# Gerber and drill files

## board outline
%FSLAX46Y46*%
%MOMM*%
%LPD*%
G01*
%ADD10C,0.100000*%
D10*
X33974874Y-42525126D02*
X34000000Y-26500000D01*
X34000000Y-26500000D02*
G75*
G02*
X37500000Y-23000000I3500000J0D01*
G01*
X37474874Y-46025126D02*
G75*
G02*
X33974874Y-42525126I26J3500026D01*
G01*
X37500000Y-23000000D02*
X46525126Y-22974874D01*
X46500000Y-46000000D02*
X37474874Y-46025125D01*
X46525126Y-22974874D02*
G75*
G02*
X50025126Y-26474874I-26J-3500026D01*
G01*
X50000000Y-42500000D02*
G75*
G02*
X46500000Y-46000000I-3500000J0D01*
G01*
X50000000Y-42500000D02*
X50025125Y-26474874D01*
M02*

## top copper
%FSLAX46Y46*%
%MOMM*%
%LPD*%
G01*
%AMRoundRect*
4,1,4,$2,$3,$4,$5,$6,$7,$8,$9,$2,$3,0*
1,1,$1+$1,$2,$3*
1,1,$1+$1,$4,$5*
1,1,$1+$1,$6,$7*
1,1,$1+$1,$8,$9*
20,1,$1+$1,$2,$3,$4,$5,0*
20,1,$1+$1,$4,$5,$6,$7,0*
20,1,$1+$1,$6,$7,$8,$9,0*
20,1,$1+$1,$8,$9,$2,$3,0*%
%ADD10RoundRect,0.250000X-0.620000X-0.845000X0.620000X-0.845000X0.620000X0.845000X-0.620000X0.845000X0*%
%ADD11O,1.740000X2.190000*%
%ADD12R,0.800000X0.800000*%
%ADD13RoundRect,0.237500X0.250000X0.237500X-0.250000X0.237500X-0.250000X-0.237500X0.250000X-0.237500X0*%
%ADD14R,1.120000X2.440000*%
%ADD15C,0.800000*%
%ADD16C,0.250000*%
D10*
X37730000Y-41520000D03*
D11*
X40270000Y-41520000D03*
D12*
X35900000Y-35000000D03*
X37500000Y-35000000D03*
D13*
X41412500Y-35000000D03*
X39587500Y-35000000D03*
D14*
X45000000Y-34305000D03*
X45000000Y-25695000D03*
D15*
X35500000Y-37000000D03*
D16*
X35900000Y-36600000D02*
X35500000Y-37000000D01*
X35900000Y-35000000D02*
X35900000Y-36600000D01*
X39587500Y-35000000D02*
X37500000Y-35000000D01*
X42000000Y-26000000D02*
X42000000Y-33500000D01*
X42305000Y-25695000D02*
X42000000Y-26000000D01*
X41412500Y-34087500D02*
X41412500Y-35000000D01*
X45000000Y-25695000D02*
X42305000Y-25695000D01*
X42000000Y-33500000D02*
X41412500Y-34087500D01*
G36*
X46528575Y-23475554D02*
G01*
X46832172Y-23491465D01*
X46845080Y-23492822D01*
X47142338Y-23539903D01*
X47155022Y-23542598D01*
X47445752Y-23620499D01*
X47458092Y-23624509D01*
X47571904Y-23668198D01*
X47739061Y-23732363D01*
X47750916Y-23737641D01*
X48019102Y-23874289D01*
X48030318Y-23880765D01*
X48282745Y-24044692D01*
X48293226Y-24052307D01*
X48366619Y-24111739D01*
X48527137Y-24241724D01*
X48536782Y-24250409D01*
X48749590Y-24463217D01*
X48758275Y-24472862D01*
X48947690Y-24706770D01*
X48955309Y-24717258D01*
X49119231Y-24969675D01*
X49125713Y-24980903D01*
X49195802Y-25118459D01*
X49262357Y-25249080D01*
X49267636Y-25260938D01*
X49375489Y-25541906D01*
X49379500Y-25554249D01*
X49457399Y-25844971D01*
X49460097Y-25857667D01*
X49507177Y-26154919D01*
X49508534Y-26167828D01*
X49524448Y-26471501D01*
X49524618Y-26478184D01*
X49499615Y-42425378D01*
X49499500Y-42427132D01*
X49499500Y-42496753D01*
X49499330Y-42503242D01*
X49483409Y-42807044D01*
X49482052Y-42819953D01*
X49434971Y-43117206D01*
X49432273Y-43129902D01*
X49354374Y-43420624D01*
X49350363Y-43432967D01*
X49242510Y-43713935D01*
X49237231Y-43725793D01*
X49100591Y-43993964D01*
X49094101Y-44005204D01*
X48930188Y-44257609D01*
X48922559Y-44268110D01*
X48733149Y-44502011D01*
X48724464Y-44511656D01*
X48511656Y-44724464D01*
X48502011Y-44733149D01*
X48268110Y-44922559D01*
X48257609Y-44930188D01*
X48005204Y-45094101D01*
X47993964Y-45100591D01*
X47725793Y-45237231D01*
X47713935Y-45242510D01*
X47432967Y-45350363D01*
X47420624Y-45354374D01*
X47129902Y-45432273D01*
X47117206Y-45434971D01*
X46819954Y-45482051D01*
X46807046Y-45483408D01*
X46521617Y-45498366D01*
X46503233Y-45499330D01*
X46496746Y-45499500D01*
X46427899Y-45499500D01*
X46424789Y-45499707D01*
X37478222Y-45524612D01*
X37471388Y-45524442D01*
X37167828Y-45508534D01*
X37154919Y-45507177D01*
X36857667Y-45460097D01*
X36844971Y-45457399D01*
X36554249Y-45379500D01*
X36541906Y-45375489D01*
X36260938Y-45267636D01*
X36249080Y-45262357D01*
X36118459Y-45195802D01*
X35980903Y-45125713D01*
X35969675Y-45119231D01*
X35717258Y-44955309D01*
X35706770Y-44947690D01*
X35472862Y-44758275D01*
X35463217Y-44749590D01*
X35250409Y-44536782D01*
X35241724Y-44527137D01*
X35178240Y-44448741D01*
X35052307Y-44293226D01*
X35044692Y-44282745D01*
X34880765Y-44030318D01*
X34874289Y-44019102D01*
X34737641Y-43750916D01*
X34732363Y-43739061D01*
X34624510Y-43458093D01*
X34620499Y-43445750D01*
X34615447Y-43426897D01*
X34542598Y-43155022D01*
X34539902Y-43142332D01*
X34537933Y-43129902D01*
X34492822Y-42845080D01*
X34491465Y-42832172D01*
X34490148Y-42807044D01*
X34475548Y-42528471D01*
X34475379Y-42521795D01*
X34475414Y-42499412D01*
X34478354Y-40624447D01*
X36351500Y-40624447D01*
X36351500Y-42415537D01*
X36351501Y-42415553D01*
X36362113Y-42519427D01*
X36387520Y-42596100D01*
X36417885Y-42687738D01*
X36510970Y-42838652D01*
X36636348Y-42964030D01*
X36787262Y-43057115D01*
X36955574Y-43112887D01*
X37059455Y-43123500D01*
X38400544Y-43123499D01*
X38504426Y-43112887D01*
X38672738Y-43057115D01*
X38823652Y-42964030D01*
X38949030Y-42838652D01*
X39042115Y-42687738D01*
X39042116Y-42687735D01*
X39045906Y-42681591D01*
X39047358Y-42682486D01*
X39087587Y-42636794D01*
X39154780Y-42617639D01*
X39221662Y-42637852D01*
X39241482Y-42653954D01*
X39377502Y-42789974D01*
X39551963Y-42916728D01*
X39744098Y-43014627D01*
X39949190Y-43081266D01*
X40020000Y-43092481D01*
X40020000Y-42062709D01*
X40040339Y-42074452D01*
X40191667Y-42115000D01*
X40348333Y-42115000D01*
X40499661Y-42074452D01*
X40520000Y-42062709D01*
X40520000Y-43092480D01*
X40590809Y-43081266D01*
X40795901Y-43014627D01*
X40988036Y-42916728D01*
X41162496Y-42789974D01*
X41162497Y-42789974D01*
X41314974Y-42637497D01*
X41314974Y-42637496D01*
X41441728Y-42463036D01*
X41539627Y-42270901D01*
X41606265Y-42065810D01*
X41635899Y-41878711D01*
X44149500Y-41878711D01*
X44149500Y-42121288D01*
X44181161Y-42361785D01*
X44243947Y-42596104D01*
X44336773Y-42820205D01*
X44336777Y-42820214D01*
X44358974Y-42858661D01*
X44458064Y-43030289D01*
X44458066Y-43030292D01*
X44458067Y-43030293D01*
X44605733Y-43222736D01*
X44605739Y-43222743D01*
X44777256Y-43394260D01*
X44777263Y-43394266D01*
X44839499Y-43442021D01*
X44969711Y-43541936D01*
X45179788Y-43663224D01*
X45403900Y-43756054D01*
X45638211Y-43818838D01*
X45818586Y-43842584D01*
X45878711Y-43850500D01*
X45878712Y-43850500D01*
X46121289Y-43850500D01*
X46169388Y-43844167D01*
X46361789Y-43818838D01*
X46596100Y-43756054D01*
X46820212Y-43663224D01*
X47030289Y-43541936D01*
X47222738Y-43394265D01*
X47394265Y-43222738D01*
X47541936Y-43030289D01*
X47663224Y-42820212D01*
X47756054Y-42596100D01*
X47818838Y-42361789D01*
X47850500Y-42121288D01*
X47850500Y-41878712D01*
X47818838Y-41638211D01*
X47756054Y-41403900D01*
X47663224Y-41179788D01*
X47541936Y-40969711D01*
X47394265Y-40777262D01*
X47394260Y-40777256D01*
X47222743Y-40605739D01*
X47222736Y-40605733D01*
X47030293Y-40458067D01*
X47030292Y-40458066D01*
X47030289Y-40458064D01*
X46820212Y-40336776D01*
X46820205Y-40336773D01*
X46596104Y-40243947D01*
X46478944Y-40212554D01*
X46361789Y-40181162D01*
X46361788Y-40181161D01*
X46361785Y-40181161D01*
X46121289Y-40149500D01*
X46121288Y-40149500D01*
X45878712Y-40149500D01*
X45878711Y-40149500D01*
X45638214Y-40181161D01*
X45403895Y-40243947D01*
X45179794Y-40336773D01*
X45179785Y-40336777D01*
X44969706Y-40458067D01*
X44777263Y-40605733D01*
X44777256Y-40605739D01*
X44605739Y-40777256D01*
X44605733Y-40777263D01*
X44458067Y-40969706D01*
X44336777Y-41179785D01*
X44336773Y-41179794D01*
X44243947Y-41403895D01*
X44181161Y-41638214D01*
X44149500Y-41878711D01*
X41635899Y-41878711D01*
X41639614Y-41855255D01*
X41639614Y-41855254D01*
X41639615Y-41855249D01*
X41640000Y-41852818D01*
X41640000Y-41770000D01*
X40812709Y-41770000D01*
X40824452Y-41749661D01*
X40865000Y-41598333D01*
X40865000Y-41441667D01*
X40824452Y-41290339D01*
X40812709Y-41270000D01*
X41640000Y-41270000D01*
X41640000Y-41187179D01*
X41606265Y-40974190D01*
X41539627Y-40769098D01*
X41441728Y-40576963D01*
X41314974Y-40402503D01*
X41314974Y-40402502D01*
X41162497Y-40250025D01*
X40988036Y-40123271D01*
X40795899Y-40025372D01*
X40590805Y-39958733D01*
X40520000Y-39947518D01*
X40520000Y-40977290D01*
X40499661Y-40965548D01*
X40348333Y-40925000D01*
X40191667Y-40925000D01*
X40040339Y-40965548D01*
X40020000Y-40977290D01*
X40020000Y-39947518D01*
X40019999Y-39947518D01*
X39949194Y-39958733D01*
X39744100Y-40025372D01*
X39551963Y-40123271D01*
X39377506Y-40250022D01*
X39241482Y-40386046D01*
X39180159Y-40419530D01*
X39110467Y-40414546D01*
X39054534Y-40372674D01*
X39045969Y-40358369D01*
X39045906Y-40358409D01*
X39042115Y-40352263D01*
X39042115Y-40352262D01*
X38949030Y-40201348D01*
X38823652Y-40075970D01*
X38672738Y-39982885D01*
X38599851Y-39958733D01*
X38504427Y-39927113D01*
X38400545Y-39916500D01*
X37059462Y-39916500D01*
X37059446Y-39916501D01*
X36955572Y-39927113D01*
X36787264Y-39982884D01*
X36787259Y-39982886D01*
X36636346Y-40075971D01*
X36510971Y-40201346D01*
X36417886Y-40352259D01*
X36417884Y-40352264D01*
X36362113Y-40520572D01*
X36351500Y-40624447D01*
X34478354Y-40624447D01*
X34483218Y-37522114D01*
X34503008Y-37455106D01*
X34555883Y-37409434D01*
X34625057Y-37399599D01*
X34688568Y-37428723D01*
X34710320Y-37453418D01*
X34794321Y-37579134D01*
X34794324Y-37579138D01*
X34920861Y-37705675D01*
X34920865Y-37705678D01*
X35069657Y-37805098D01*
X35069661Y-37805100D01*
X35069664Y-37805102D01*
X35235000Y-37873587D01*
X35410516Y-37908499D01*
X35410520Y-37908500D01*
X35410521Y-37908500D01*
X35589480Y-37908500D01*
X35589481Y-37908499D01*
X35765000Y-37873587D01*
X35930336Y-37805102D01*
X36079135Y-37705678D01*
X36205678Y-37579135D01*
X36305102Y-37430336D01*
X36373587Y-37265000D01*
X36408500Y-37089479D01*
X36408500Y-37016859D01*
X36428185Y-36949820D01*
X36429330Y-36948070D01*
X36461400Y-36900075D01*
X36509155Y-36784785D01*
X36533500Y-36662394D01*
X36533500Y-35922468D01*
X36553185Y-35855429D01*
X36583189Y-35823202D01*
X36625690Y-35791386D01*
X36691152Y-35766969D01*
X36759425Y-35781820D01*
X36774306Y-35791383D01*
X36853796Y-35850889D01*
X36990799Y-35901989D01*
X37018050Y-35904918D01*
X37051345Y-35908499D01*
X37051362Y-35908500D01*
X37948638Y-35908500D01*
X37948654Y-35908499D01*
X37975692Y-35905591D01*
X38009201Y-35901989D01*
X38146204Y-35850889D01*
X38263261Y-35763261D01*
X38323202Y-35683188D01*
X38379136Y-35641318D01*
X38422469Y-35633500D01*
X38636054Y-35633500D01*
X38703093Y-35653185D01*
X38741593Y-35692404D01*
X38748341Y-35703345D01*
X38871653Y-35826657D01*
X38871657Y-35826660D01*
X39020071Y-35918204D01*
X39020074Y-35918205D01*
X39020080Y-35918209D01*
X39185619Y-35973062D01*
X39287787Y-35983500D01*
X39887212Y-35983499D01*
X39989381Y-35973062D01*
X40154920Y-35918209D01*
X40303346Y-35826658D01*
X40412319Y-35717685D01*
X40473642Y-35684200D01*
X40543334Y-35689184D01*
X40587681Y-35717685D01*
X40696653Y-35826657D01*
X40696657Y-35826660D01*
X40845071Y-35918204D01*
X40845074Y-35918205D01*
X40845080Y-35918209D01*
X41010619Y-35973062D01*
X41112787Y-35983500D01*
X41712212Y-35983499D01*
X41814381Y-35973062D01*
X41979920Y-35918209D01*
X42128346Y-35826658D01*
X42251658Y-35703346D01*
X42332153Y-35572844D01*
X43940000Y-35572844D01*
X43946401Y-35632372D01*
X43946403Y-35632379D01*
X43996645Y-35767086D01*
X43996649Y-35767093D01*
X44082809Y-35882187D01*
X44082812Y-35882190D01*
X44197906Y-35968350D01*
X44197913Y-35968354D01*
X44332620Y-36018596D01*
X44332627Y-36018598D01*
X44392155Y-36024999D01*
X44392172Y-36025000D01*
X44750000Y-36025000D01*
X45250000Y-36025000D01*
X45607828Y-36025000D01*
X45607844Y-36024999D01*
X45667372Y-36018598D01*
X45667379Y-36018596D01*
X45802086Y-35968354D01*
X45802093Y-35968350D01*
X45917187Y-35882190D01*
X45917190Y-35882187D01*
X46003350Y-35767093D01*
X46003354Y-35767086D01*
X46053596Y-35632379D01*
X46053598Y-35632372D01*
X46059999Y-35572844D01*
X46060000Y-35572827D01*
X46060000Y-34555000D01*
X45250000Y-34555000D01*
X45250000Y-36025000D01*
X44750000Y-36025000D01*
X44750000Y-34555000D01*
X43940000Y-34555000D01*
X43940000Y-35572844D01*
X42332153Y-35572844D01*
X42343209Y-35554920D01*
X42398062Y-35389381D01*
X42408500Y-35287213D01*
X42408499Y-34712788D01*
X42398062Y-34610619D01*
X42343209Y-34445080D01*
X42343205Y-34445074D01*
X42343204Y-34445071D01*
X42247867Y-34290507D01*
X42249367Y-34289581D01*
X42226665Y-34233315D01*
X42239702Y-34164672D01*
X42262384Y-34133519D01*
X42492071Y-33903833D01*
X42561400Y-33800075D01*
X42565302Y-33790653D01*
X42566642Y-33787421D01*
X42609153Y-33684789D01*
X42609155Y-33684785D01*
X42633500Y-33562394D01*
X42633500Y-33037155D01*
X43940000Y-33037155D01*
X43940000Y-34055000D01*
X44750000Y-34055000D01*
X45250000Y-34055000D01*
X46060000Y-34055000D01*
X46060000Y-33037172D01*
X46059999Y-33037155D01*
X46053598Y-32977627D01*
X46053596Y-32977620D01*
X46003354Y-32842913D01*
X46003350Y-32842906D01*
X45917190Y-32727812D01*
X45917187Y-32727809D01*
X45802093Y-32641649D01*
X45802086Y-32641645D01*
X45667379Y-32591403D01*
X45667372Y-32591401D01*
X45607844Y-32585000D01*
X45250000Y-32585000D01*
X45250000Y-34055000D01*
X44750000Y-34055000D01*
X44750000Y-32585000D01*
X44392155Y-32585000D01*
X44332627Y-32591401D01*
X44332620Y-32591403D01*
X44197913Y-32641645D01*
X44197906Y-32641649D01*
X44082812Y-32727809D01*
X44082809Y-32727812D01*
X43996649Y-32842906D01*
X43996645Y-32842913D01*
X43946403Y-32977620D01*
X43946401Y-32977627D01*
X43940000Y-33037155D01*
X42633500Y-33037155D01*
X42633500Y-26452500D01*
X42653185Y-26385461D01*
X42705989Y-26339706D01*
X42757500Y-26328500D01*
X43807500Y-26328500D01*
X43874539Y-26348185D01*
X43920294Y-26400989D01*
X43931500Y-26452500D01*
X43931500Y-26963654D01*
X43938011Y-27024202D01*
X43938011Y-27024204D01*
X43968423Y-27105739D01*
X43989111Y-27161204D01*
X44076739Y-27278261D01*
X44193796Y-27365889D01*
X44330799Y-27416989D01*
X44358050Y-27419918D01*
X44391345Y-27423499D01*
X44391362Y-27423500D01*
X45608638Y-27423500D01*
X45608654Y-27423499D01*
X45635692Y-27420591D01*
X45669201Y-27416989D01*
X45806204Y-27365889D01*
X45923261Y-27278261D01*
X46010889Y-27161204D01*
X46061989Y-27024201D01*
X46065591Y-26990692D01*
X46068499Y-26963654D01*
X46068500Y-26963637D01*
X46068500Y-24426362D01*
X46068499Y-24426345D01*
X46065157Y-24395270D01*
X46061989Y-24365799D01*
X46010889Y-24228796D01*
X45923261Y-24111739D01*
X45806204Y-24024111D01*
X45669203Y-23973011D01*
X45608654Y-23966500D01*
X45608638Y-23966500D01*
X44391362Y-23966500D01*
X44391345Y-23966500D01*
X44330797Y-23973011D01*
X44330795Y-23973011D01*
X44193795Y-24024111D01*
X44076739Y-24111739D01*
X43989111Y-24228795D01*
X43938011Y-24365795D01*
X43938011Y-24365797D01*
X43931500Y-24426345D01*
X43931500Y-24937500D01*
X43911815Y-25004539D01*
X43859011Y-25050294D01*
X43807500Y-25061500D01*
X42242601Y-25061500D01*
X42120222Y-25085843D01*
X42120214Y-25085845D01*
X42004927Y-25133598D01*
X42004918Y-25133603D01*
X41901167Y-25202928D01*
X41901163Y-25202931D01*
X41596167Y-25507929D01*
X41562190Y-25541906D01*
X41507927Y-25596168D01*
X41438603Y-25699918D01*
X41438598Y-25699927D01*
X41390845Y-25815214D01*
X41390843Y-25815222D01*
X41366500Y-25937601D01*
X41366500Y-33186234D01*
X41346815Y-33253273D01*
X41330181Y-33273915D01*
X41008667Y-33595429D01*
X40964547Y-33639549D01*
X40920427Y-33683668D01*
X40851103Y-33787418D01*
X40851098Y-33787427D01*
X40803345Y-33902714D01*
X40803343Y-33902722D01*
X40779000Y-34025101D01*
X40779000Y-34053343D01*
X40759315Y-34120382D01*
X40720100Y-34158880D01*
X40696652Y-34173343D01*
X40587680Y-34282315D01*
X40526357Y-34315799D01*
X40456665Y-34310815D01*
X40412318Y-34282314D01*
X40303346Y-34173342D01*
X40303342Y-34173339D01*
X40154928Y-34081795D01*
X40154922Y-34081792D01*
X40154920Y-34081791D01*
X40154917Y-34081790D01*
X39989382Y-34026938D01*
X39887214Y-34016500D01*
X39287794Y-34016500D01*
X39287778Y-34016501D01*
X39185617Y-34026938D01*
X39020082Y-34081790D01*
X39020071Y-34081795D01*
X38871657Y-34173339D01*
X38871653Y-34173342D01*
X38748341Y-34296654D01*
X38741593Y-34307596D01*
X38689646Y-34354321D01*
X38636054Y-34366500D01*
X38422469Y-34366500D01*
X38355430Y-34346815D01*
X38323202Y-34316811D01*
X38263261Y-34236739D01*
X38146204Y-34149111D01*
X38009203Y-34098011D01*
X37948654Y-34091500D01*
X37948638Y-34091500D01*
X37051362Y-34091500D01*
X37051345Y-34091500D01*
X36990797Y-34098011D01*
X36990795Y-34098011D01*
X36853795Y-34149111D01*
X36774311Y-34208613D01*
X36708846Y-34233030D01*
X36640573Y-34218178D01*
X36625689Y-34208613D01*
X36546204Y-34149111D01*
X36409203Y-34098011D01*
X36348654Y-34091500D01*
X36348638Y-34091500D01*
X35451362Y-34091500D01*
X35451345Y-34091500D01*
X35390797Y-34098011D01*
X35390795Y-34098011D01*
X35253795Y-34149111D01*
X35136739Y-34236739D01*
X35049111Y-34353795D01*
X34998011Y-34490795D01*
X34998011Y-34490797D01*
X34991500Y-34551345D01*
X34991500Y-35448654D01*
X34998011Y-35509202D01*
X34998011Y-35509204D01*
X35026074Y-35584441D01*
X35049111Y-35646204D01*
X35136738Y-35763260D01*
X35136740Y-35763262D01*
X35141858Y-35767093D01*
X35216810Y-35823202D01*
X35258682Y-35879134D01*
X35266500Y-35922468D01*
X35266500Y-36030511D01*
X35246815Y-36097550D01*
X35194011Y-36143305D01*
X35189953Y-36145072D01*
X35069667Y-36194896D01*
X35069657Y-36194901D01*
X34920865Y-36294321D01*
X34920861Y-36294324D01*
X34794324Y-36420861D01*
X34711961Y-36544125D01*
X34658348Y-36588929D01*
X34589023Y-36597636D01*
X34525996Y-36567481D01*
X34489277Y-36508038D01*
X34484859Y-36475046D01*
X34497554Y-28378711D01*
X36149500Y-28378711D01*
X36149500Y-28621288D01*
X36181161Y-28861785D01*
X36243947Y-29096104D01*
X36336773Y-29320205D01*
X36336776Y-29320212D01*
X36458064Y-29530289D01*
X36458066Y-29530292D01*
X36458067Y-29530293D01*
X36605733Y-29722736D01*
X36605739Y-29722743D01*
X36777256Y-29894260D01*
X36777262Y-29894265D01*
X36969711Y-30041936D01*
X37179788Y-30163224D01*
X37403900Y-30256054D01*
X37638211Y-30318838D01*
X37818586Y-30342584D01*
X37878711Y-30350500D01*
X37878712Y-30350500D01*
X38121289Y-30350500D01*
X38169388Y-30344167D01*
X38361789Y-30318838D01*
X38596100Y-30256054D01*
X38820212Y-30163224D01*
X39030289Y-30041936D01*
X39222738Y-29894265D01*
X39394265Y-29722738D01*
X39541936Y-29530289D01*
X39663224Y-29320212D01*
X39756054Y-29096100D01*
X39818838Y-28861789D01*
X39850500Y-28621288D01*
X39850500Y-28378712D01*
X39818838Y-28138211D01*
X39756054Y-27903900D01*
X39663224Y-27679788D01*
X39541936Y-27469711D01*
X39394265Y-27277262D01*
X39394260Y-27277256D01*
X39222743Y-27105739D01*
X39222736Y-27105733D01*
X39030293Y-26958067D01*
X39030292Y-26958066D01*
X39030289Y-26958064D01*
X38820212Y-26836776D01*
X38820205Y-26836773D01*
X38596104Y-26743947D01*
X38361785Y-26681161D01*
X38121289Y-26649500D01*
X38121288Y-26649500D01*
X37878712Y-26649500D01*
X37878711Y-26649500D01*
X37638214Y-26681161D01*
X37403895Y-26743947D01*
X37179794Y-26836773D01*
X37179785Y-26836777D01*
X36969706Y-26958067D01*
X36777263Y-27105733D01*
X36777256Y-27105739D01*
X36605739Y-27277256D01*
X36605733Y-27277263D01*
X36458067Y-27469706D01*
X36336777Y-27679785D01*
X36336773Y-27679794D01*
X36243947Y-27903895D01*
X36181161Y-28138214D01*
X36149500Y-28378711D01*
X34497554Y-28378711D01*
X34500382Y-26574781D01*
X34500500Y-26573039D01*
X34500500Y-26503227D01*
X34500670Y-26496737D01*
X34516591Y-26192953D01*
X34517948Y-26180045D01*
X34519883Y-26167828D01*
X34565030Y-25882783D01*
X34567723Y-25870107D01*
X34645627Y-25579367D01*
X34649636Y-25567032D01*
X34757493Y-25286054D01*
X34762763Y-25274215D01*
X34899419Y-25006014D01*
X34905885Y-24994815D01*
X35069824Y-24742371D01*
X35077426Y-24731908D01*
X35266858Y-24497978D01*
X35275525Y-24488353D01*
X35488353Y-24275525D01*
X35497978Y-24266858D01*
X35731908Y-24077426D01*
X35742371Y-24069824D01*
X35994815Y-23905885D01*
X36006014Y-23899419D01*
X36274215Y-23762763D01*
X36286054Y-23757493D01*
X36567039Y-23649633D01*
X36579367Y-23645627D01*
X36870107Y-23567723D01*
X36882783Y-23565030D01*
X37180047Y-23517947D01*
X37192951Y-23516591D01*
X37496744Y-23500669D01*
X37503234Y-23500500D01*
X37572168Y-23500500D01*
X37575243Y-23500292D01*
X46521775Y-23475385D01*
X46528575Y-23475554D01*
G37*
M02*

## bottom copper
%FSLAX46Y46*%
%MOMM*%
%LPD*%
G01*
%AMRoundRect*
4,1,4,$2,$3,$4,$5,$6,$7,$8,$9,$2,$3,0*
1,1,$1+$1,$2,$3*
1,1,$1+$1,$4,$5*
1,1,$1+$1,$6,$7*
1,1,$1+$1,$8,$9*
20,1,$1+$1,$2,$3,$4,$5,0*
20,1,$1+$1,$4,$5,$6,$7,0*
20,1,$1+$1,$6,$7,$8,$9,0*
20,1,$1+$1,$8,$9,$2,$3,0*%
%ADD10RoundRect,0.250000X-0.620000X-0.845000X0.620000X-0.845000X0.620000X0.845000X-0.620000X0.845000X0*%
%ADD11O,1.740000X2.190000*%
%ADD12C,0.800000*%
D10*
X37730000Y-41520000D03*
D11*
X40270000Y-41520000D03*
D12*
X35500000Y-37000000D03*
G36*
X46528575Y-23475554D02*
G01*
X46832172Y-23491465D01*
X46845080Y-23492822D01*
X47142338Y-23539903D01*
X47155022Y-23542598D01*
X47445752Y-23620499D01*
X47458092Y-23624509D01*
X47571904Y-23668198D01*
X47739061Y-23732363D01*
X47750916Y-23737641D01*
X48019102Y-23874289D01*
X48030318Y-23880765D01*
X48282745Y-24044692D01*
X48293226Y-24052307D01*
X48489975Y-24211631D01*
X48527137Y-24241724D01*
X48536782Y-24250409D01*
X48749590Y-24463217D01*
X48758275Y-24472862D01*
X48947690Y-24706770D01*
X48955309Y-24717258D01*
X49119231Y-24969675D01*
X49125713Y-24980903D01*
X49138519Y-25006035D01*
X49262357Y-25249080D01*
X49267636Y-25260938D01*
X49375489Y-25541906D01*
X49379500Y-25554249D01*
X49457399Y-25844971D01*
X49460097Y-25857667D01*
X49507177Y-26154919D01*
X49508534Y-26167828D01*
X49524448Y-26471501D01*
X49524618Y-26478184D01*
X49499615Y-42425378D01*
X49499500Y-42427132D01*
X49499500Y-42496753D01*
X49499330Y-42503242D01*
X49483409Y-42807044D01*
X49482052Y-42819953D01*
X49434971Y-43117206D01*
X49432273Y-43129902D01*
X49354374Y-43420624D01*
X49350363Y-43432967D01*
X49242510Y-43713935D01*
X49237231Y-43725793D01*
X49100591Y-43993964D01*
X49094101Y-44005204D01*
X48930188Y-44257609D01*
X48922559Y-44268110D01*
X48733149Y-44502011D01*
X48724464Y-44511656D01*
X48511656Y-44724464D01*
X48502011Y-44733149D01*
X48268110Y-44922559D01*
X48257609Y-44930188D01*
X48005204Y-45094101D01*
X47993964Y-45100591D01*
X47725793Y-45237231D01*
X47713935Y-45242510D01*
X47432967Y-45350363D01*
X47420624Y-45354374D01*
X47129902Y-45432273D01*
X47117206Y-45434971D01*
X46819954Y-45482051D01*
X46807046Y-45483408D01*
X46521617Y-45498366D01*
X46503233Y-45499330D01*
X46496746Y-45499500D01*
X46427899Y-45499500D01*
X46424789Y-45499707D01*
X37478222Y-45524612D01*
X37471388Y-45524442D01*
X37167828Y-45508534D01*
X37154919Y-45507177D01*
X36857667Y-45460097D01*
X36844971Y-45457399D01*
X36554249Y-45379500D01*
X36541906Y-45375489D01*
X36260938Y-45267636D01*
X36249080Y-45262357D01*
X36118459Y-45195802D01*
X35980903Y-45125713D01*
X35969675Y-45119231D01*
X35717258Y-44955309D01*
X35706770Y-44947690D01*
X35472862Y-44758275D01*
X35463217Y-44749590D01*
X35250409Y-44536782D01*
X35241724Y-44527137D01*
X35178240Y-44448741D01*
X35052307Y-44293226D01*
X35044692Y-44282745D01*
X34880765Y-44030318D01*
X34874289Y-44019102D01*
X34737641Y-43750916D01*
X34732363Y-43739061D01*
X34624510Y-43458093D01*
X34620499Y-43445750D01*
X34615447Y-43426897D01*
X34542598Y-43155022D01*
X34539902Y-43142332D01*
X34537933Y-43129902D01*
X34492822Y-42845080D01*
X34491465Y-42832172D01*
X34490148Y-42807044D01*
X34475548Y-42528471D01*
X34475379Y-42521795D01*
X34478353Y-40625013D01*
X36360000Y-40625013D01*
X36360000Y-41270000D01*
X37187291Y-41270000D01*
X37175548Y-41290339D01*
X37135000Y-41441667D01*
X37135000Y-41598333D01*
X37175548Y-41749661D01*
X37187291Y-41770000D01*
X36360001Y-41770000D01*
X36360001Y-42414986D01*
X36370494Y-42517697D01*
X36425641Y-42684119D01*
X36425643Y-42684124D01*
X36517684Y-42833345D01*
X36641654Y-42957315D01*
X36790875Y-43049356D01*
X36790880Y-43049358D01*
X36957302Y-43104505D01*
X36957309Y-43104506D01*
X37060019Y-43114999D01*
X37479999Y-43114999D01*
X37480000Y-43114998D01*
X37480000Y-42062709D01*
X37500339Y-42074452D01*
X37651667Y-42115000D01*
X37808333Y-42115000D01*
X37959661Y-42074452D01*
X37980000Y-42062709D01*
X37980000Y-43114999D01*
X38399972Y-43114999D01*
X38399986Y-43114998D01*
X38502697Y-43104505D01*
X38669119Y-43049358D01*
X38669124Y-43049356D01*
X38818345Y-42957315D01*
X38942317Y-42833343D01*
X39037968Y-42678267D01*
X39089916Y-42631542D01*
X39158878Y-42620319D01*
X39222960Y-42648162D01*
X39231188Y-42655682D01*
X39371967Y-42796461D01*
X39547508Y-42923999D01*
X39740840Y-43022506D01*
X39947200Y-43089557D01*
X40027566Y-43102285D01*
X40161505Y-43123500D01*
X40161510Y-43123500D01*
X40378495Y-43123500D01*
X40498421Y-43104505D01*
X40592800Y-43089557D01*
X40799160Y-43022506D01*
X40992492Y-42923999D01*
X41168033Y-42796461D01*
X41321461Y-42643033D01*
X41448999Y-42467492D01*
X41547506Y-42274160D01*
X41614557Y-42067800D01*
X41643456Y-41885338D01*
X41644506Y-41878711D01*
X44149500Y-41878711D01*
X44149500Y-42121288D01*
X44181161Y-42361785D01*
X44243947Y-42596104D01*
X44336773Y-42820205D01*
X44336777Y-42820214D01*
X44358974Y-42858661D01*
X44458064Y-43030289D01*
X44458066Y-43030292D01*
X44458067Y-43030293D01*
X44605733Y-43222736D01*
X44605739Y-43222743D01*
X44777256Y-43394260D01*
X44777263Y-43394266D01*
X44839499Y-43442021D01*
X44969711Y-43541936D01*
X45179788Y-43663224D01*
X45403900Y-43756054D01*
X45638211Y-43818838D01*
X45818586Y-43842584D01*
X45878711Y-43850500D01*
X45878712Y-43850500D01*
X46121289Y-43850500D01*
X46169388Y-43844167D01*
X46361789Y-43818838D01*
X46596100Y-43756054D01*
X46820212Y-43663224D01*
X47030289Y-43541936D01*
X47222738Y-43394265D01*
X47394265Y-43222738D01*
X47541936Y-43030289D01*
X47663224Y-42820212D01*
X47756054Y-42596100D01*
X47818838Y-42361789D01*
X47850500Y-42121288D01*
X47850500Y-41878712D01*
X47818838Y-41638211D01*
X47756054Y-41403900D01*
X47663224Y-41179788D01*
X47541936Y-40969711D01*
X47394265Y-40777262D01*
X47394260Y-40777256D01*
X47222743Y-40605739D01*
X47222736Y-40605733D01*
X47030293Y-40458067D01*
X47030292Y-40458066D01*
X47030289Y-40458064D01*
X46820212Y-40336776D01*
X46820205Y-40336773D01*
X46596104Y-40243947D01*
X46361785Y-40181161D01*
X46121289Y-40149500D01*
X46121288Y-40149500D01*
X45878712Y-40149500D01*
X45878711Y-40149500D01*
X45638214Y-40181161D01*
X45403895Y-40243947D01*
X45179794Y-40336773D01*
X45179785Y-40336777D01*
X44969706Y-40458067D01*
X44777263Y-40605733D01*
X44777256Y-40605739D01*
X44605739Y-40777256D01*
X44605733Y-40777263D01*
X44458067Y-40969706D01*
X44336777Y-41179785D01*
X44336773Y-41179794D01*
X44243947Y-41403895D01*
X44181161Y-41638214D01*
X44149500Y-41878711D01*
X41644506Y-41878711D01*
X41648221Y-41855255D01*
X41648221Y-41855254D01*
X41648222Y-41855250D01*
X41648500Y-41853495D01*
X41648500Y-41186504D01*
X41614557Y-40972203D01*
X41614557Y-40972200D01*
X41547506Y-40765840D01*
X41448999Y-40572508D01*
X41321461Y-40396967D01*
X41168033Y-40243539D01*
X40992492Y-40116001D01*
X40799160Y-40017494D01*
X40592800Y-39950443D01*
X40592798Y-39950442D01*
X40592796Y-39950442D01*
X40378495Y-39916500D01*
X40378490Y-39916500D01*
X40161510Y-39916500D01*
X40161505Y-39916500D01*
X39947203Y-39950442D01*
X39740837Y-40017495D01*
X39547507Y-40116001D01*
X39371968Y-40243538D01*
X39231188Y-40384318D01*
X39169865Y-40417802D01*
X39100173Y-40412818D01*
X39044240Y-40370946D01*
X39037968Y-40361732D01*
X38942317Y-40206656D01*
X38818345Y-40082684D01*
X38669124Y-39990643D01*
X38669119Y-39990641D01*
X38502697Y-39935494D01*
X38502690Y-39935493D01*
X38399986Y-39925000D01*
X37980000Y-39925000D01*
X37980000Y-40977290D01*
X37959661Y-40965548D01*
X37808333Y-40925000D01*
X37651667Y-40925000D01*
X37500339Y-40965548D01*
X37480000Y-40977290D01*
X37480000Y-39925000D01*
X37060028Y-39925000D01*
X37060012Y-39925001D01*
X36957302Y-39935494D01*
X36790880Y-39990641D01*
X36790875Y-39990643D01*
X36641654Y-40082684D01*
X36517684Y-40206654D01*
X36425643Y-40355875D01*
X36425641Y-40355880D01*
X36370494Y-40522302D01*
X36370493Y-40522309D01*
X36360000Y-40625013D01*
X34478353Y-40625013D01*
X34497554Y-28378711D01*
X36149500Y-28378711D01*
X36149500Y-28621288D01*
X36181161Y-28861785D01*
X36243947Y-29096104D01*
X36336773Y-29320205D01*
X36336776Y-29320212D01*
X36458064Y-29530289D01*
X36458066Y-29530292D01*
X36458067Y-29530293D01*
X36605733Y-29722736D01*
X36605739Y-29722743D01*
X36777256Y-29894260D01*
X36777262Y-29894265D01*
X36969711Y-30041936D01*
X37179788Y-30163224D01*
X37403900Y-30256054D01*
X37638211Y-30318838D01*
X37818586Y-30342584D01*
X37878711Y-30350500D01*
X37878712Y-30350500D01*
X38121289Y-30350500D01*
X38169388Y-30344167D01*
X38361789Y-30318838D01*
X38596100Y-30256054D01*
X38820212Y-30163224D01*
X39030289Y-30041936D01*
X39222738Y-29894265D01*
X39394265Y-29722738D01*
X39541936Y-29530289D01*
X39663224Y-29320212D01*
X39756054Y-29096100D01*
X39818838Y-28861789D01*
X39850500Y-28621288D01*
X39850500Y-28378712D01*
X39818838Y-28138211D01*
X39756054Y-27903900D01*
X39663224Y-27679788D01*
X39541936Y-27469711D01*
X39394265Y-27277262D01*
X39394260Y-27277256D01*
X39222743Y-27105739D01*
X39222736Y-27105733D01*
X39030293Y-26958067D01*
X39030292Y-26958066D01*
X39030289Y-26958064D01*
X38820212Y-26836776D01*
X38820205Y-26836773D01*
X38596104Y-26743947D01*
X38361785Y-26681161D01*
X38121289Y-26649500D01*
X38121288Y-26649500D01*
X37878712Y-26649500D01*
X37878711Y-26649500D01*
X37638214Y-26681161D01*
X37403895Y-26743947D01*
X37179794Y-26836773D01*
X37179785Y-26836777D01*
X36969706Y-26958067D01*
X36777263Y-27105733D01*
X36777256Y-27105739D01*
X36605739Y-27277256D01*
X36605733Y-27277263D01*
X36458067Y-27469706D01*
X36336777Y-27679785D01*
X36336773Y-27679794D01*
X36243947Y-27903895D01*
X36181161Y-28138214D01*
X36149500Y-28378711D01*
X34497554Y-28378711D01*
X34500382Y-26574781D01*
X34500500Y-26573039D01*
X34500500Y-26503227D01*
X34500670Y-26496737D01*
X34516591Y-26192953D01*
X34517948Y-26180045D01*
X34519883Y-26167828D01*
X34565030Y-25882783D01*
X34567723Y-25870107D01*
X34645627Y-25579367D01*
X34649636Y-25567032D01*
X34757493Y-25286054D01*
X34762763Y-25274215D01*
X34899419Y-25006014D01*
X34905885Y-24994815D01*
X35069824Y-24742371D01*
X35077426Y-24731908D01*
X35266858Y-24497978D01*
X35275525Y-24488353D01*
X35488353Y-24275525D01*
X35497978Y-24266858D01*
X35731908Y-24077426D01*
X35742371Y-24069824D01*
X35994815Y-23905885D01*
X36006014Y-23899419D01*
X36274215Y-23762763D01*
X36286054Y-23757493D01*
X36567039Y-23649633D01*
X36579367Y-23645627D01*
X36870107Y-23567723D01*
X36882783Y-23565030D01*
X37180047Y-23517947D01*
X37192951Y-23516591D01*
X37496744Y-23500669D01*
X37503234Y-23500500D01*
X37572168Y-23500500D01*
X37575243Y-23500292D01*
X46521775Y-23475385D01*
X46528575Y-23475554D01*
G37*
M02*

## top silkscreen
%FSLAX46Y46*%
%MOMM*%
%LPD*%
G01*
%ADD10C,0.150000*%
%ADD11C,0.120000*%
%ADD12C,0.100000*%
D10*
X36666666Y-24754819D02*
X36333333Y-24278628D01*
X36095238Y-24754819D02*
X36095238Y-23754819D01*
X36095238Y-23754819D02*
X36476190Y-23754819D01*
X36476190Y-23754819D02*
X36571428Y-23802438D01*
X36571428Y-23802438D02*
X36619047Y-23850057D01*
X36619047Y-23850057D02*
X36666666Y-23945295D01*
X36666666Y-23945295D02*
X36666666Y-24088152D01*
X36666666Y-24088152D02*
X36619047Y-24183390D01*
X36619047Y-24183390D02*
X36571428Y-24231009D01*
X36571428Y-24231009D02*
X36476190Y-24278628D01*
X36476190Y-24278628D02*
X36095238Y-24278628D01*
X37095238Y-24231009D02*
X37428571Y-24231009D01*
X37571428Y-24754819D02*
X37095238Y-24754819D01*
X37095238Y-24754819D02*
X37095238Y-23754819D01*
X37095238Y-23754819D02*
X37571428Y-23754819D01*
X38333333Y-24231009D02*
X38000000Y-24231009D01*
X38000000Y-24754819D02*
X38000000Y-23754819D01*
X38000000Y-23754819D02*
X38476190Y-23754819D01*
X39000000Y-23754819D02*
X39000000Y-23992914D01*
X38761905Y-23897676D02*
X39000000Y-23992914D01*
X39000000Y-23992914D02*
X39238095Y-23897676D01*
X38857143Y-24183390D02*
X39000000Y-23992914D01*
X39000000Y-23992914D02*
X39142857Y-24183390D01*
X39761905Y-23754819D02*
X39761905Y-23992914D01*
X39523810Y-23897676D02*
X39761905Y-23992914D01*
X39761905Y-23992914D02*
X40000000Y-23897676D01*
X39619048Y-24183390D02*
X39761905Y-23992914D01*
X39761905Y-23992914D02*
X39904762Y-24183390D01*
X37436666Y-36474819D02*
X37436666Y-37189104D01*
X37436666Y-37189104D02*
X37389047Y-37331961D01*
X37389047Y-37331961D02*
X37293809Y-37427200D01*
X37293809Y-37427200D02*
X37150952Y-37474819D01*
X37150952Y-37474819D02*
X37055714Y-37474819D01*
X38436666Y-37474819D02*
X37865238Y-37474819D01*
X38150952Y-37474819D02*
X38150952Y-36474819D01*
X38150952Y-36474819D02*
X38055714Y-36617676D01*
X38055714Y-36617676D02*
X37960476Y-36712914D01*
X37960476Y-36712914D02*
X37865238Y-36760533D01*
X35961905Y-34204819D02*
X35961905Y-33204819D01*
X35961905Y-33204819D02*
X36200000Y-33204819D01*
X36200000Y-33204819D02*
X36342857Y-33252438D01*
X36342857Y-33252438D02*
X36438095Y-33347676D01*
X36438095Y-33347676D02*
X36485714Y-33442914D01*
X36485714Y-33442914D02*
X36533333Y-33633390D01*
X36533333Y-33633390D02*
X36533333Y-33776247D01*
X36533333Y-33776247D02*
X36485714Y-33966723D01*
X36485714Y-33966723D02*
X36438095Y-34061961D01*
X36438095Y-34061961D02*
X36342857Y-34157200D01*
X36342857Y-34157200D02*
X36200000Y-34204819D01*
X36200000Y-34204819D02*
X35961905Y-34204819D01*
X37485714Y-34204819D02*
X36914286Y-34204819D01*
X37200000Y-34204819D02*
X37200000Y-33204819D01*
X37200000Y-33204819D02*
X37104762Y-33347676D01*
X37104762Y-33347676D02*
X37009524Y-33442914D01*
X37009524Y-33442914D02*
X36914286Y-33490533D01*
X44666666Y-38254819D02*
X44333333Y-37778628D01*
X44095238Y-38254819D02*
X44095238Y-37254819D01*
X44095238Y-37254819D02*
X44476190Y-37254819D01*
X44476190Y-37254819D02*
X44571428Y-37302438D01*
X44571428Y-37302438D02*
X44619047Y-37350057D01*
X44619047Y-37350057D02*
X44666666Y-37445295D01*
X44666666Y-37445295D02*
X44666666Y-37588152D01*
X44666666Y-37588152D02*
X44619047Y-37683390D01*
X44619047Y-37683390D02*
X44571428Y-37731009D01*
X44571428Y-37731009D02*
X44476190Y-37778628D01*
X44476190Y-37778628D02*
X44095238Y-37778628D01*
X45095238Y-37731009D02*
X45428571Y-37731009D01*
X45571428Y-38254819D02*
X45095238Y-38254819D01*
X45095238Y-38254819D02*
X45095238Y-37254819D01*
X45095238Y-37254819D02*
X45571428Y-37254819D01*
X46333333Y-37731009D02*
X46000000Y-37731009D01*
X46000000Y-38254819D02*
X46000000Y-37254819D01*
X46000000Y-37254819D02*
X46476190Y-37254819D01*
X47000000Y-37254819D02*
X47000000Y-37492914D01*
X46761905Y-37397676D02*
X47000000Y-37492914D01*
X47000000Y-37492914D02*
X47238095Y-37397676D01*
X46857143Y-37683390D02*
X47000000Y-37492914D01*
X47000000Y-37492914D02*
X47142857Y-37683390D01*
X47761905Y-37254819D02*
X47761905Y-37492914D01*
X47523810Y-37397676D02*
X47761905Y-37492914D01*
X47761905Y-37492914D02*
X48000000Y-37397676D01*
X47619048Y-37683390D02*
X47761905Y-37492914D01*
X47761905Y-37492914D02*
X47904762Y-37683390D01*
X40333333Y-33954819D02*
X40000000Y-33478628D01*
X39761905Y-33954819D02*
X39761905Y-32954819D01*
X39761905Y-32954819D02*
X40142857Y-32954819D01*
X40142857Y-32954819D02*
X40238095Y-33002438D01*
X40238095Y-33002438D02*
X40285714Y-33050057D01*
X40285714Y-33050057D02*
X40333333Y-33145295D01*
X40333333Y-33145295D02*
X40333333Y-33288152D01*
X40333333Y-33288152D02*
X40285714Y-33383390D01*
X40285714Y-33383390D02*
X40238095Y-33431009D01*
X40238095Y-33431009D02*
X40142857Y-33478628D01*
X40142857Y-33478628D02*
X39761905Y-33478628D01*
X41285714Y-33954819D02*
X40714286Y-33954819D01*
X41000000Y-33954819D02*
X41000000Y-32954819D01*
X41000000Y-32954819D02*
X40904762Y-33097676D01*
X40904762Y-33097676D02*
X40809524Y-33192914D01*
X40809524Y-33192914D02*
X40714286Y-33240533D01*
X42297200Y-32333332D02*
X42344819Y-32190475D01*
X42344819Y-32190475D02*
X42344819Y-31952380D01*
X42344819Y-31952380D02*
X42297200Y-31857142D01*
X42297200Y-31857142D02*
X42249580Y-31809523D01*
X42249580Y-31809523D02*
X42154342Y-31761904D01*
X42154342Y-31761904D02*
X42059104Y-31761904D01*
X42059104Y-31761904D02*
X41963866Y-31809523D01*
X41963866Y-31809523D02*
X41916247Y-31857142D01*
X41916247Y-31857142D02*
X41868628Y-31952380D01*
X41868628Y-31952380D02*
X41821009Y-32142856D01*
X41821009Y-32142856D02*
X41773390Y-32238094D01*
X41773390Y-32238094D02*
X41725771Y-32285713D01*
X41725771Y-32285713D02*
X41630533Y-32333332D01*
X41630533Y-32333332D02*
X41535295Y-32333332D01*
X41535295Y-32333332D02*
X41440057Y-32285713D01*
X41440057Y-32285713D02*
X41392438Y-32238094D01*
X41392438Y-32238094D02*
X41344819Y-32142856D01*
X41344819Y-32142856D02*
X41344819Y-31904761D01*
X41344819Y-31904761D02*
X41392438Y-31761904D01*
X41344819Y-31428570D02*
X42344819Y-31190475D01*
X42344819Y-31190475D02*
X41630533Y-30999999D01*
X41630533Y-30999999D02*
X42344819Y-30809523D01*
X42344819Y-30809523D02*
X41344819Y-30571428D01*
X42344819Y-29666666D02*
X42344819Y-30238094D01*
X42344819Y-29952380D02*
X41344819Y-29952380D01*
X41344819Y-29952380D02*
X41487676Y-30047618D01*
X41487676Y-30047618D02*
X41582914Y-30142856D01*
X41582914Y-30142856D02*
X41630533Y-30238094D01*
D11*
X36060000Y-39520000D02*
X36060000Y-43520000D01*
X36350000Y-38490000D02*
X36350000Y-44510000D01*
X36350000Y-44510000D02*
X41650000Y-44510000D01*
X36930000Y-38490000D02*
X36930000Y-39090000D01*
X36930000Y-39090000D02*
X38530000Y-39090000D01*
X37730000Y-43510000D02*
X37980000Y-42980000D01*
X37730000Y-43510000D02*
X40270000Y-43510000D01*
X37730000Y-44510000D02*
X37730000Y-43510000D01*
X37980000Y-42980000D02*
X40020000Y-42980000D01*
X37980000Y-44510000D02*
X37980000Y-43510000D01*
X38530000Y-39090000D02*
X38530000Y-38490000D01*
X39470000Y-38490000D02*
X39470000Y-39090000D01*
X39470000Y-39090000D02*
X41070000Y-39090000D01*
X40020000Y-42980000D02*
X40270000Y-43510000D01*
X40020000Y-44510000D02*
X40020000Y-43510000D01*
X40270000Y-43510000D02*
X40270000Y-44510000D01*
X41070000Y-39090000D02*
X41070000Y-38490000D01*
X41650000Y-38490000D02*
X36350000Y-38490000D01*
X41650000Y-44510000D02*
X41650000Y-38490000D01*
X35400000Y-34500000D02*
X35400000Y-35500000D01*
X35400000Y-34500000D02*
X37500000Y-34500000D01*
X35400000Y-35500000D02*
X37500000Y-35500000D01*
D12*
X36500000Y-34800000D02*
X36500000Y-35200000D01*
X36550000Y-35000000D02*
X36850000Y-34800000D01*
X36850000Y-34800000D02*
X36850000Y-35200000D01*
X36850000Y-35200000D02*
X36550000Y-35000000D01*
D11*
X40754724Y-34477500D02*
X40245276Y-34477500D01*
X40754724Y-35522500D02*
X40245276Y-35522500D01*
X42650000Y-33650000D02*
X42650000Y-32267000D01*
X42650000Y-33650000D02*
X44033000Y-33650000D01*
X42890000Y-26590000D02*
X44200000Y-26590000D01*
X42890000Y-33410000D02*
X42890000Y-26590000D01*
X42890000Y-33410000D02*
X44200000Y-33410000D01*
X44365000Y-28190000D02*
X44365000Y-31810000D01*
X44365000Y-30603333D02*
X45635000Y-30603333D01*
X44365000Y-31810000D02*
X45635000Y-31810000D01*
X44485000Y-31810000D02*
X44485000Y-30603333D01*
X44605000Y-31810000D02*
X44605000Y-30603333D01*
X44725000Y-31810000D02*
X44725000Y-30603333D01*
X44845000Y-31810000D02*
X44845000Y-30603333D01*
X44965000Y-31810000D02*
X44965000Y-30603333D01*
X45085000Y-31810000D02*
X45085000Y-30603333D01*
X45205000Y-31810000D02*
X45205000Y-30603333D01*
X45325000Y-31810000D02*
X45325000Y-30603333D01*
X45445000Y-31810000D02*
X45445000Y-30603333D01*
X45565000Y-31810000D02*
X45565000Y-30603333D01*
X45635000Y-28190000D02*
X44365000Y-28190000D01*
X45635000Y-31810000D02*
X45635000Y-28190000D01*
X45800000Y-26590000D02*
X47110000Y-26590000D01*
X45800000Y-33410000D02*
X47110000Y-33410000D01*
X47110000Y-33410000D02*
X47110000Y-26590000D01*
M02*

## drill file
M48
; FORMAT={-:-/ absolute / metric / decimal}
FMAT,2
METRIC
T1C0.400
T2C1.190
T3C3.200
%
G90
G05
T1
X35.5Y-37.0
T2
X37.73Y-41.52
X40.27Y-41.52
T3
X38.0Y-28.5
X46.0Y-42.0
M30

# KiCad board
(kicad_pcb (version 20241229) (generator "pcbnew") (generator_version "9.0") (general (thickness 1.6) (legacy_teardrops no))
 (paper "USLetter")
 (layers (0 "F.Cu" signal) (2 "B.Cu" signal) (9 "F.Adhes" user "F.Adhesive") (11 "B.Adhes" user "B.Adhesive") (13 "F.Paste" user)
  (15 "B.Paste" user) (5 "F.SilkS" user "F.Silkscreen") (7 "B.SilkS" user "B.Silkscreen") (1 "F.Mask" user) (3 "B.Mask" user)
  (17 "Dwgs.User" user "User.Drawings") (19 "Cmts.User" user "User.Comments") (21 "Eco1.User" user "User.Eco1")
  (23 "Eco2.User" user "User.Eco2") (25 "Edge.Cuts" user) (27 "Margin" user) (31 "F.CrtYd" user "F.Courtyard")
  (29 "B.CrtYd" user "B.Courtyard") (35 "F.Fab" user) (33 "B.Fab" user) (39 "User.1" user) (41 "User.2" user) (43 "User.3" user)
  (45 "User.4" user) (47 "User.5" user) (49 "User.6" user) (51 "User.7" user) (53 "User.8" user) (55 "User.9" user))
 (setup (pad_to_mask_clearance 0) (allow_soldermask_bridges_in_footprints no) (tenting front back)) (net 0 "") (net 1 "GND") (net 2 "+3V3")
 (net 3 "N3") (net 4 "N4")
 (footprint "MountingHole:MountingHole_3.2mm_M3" (layer "F.Cu") (at 38 28.5)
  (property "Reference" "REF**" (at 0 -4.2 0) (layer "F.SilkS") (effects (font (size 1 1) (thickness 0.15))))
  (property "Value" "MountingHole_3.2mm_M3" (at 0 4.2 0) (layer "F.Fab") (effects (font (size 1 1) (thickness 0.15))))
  (pad "" np_thru_hole circle (at 0 0) (size 3.2 3.2) (drill 3.2) (layers "*.Cu" "*.Mask")))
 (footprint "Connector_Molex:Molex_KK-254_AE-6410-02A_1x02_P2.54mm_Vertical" (layer "F.Cu") (at 37.73 41.52)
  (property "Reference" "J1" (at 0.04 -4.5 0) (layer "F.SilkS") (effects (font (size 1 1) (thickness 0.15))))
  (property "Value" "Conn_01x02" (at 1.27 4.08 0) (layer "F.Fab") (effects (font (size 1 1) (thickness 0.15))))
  (fp_line (start -1.67 -2) (end -1.67 2) (stroke (width 0.12) (type solid)) (layer "F.SilkS"))
  (fp_line (start -1.38 -3.03) (end -1.38 2.99) (stroke (width 0.12) (type solid)) (layer "F.SilkS"))
  (fp_line (start -1.38 2.99) (end 3.92 2.99) (stroke (width 0.12) (type solid)) (layer "F.SilkS"))
  (fp_line (start -0.8 -3.03) (end -0.8 -2.43) (stroke (width 0.12) (type solid)) (layer "F.SilkS"))
  (fp_line (start -0.8 -2.43) (end 0.8 -2.43) (stroke (width 0.12) (type solid)) (layer "F.SilkS"))
  (fp_line (start 0 1.99) (end 0.25 1.46) (stroke (width 0.12) (type solid)) (layer "F.SilkS"))
  (fp_line (start 0 1.99) (end 2.54 1.99) (stroke (width 0.12) (type solid)) (layer "F.SilkS"))
  (fp_line (start 0 2.99) (end 0 1.99) (stroke (width 0.12) (type solid)) (layer "F.SilkS"))
  (fp_line (start 0.25 1.46) (end 2.29 1.46) (stroke (width 0.12) (type solid)) (layer "F.SilkS"))
  (fp_line (start 0.25 2.99) (end 0.25 1.99) (stroke (width 0.12) (type solid)) (layer "F.SilkS"))
  (fp_line (start 0.8 -2.43) (end 0.8 -3.03) (stroke (width 0.12) (type solid)) (layer "F.SilkS"))
  (fp_line (start 1.74 -3.03) (end 1.74 -2.43) (stroke (width 0.12) (type solid)) (layer "F.SilkS"))
  (fp_line (start 1.74 -2.43) (end 3.34 -2.43) (stroke (width 0.12) (type solid)) (layer "F.SilkS"))
  (fp_line (start 2.29 1.46) (end 2.54 1.99) (stroke (width 0.12) (type solid)) (layer "F.SilkS"))
  (fp_line (start 2.29 2.99) (end 2.29 1.99) (stroke (width 0.12) (type solid)) (layer "F.SilkS"))
  (fp_line (start 2.54 1.99) (end 2.54 2.99) (stroke (width 0.12) (type solid)) (layer "F.SilkS"))
  (fp_line (start 3.34 -2.43) (end 3.34 -3.03) (stroke (width 0.12) (type solid)) (layer "F.SilkS"))
  (fp_line (start 3.92 -3.03) (end -1.38 -3.03) (stroke (width 0.12) (type solid)) (layer "F.SilkS"))
  (fp_line (start 3.92 2.99) (end 3.92 -3.03) (stroke (width 0.12) (type solid)) (layer "F.SilkS"))
  (pad "1" thru_hole roundrect (at 0 0) (size 1.74 2.19) (drill 1.19) (layers "*.Cu" "*.Mask") (remove_unused_layers no)
   (roundrect_rratio 0.143678) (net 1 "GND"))
  (pad "2" thru_hole oval (at 2.54 0) (size 1.74 2.19) (drill 1.19) (layers "*.Cu" "*.Mask") (remove_unused_layers no) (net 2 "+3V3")))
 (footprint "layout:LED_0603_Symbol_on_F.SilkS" (layer "F.Cu") (at 36.7 35)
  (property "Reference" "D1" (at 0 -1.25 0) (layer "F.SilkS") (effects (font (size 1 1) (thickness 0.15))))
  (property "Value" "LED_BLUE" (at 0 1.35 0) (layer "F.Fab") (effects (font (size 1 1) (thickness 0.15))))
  (fp_line (start -1.3 -0.5) (end -1.3 0.5) (stroke (width 0.12) (type solid)) (layer "F.SilkS"))
  (fp_line (start -1.3 -0.5) (end 0.8 -0.5) (stroke (width 0.12) (type solid)) (layer "F.SilkS"))
  (fp_line (start -1.3 0.5) (end 0.8 0.5) (stroke (width 0.12) (type solid)) (layer "F.SilkS"))
  (fp_line (start -0.2 -0.2) (end -0.2 0.2) (stroke (width 0.1) (type solid)) (layer "F.SilkS"))
  (fp_line (start -0.15 0) (end 0.15 -0.2) (stroke (width 0.1) (type solid)) (layer "F.SilkS"))
  (fp_line (start 0.15 -0.2) (end 0.15 0.2) (stroke (width 0.1) (type solid)) (layer "F.SilkS"))
  (fp_line (start 0.15 0.2) (end -0.15 0) (stroke (width 0.1) (type solid)) (layer "F.SilkS"))
  (pad "1" smd rect (at -0.8 0 180) (size 0.8 0.8) (layers "F.Cu" "F.Mask" "F.Paste") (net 1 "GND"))
  (pad "2" smd rect (at 0.8 0 180) (size 0.8 0.8) (layers "F.Cu" "F.Mask" "F.Paste") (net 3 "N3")))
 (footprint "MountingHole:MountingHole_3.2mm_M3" (layer "F.Cu") (at 46 42)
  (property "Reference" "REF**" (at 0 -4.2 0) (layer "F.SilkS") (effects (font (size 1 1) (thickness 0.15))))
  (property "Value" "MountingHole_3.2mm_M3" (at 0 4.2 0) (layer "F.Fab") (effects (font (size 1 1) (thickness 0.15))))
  (pad "" np_thru_hole circle (at 0 0) (size 3.2 3.2) (drill 3.2) (layers "*.Cu" "*.Mask")))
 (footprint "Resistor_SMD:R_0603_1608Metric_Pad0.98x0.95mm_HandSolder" (layer "F.Cu") (at 40.5 35 180)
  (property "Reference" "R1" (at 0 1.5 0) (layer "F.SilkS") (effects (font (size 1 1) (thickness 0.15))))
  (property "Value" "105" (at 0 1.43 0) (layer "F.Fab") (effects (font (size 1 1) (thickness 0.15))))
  (fp_line (start -0.254724 0.5225) (end 0.254724 0.5225) (stroke (width 0.12) (type solid)) (layer "F.SilkS"))
  (fp_line (start -0.254724 -0.5225) (end 0.254724 -0.5225) (stroke (width 0.12) (type solid)) (layer "F.SilkS"))
  (pad "1" smd roundrect (at -0.9125 0 180) (size 0.975 0.95) (layers "F.Cu" "F.Mask" "F.Paste") (roundrect_rratio 0.25) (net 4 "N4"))
  (pad "2" smd roundrect (at 0.9125 0 180) (size 0.975 0.95) (layers "F.Cu" "F.Mask" "F.Paste") (roundrect_rratio 0.25) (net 3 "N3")))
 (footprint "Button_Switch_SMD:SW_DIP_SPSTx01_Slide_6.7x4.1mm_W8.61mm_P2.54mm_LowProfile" (layer "F.Cu") (at 45 30 90)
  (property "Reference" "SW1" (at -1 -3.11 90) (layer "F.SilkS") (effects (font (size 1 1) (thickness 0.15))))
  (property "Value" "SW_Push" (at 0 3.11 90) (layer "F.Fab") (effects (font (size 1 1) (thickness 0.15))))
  (fp_line (start -3.65 -2.35) (end -2.267 -2.35) (stroke (width 0.12) (type solid)) (layer "F.SilkS"))
  (fp_line (start -3.65 -2.35) (end -3.65 -0.967) (stroke (width 0.12) (type solid)) (layer "F.SilkS"))
  (fp_line (start 3.41 -2.11) (end 3.41 -0.8) (stroke (width 0.12) (type solid)) (layer "F.SilkS"))
  (fp_line (start -3.41 -2.11) (end 3.41 -2.11) (stroke (width 0.12) (type solid)) (layer "F.SilkS"))
  (fp_line (start -3.41 -2.11) (end -3.41 -0.8) (stroke (width 0.12) (type solid)) (layer "F.SilkS"))
  (fp_line (start 1.81 -0.635) (end -1.81 -0.635) (stroke (width 0.12) (type solid)) (layer "F.SilkS"))
  (fp_line (start -0.603333 -0.635) (end -0.603333 0.635) (stroke (width 0.12) (type solid)) (layer "F.SilkS"))
  (fp_line (start -1.81 -0.635) (end -1.81 0.635) (stroke (width 0.12) (type solid)) (layer "F.SilkS"))
  (fp_line (start -1.81 -0.515) (end -0.603333 -0.515) (stroke (width 0.12) (type solid)) (layer "F.SilkS"))
  (fp_line (start -1.81 -0.395) (end -0.603333 -0.395) (stroke (width 0.12) (type solid)) (layer "F.SilkS"))
  (fp_line (start -1.81 -0.275) (end -0.603333 -0.275) (stroke (width 0.12) (type solid)) (layer "F.SilkS"))
  (fp_line (start -1.81 -0.155) (end -0.603333 -0.155) (stroke (width 0.12) (type solid)) (layer "F.SilkS"))
  (fp_line (start -1.81 -0.035) (end -0.603333 -0.035) (stroke (width 0.12) (type solid)) (layer "F.SilkS"))
  (fp_line (start -1.81 0.085) (end -0.603333 0.085) (stroke (width 0.12) (type solid)) (layer "F.SilkS"))
  (fp_line (start -1.81 0.205) (end -0.603333 0.205) (stroke (width 0.12) (type solid)) (layer "F.SilkS"))
  (fp_line (start -1.81 0.325) (end -0.603333 0.325) (stroke (width 0.12) (type solid)) (layer "F.SilkS"))
  (fp_line (start -1.81 0.445) (end -0.603333 0.445) (stroke (width 0.12) (type solid)) (layer "F.SilkS"))
  (fp_line (start -1.81 0.565) (end -0.603333 0.565) (stroke (width 0.12) (type solid)) (layer "F.SilkS"))
  (fp_line (start 1.81 0.635) (end 1.81 -0.635) (stroke (width 0.12) (type solid)) (layer "F.SilkS"))
  (fp_line (start -1.81 0.635) (end 1.81 0.635) (stroke (width 0.12) (type solid)) (layer "F.SilkS"))
  (fp_line (start 3.41 0.8) (end 3.41 2.11) (stroke (width 0.12) (type solid)) (layer "F.SilkS"))
  (fp_line (start -3.41 0.8) (end -3.41 2.11) (stroke (width 0.12) (type solid)) (layer "F.SilkS"))
  (fp_line (start -3.41 2.11) (end 3.41 2.11) (stroke (width 0.12) (type solid)) (layer "F.SilkS"))
  (pad "1" smd rect (at -4.305 0 90) (size 2.44 1.12) (layers "F.Cu" "F.Mask" "F.Paste") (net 2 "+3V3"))
  (pad "2" smd rect (at 4.305 0 90) (size 2.44 1.12) (layers "F.Cu" "F.Mask" "F.Paste") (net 4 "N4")))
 (gr_line (start 33.974874 42.525126) (end 34 26.5) (stroke (width 0.1) (type default)) (layer "Edge.Cuts"))
 (gr_arc (start 34 26.5) (mid 35.025126 24.025126) (end 37.5 23) (stroke (width 0.1) (type default)) (layer "Edge.Cuts"))
 (gr_arc (start 37.474874 46.025126) (mid 35 45) (end 33.974874 42.525126) (stroke (width 0.1) (type default)) (layer "Edge.Cuts"))
 (gr_line (start 37.5 23) (end 46.525126 22.974874) (stroke (width 0.1) (type default)) (layer "Edge.Cuts"))
 (gr_line (start 46.5 46) (end 37.474874 46.025125) (stroke (width 0.1) (type default)) (layer "Edge.Cuts"))
 (gr_arc (start 46.525126 22.974874) (mid 49 24) (end 50.025126 26.474874) (stroke (width 0.1) (type default)) (layer "Edge.Cuts"))
 (gr_arc (start 50 42.5) (mid 48.974874 44.974874) (end 46.5 46) (stroke (width 0.1) (type default)) (layer "Edge.Cuts"))
 (gr_line (start 50 42.5) (end 50.025125 26.474874) (stroke (width 0.1) (type default)) (layer "Edge.Cuts"))
 (segment (start 35.9 36.6) (end 35.5 37) (width 0.25) (layer "F.Cu") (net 1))
 (segment (start 35.9 35) (end 35.9 36.6) (width 0.25) (layer "F.Cu") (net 1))
 (via (at 35.5 37) (size 0.8) (drill 0.4) (layers "F.Cu" "B.Cu") (free yes) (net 1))
 (segment (start 39.5875 35) (end 37.5 35) (width 0.25) (layer "F.Cu") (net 3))
 (segment (start 42 26) (end 42 33.5) (width 0.25) (layer "F.Cu") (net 4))
 (segment (start 42.305 25.695) (end 42 26) (width 0.25) (layer "F.Cu") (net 4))
 (segment (start 41.4125 34.0875) (end 41.4125 35) (width 0.25) (layer "F.Cu") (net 4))
 (segment (start 45 25.695) (end 42.305 25.695) (width 0.25) (layer "F.Cu") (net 4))
 (segment (start 42 33.5) (end 41.4125 34.0875) (width 0.25) (layer "F.Cu") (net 4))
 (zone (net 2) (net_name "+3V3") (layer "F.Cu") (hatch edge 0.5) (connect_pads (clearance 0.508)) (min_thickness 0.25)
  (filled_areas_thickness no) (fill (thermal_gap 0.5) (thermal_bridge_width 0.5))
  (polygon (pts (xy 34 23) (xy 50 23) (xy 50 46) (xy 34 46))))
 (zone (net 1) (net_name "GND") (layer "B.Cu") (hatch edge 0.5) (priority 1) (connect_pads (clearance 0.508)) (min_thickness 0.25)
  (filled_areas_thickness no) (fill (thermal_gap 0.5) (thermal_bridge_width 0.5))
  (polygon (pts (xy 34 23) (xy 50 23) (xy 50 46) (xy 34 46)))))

